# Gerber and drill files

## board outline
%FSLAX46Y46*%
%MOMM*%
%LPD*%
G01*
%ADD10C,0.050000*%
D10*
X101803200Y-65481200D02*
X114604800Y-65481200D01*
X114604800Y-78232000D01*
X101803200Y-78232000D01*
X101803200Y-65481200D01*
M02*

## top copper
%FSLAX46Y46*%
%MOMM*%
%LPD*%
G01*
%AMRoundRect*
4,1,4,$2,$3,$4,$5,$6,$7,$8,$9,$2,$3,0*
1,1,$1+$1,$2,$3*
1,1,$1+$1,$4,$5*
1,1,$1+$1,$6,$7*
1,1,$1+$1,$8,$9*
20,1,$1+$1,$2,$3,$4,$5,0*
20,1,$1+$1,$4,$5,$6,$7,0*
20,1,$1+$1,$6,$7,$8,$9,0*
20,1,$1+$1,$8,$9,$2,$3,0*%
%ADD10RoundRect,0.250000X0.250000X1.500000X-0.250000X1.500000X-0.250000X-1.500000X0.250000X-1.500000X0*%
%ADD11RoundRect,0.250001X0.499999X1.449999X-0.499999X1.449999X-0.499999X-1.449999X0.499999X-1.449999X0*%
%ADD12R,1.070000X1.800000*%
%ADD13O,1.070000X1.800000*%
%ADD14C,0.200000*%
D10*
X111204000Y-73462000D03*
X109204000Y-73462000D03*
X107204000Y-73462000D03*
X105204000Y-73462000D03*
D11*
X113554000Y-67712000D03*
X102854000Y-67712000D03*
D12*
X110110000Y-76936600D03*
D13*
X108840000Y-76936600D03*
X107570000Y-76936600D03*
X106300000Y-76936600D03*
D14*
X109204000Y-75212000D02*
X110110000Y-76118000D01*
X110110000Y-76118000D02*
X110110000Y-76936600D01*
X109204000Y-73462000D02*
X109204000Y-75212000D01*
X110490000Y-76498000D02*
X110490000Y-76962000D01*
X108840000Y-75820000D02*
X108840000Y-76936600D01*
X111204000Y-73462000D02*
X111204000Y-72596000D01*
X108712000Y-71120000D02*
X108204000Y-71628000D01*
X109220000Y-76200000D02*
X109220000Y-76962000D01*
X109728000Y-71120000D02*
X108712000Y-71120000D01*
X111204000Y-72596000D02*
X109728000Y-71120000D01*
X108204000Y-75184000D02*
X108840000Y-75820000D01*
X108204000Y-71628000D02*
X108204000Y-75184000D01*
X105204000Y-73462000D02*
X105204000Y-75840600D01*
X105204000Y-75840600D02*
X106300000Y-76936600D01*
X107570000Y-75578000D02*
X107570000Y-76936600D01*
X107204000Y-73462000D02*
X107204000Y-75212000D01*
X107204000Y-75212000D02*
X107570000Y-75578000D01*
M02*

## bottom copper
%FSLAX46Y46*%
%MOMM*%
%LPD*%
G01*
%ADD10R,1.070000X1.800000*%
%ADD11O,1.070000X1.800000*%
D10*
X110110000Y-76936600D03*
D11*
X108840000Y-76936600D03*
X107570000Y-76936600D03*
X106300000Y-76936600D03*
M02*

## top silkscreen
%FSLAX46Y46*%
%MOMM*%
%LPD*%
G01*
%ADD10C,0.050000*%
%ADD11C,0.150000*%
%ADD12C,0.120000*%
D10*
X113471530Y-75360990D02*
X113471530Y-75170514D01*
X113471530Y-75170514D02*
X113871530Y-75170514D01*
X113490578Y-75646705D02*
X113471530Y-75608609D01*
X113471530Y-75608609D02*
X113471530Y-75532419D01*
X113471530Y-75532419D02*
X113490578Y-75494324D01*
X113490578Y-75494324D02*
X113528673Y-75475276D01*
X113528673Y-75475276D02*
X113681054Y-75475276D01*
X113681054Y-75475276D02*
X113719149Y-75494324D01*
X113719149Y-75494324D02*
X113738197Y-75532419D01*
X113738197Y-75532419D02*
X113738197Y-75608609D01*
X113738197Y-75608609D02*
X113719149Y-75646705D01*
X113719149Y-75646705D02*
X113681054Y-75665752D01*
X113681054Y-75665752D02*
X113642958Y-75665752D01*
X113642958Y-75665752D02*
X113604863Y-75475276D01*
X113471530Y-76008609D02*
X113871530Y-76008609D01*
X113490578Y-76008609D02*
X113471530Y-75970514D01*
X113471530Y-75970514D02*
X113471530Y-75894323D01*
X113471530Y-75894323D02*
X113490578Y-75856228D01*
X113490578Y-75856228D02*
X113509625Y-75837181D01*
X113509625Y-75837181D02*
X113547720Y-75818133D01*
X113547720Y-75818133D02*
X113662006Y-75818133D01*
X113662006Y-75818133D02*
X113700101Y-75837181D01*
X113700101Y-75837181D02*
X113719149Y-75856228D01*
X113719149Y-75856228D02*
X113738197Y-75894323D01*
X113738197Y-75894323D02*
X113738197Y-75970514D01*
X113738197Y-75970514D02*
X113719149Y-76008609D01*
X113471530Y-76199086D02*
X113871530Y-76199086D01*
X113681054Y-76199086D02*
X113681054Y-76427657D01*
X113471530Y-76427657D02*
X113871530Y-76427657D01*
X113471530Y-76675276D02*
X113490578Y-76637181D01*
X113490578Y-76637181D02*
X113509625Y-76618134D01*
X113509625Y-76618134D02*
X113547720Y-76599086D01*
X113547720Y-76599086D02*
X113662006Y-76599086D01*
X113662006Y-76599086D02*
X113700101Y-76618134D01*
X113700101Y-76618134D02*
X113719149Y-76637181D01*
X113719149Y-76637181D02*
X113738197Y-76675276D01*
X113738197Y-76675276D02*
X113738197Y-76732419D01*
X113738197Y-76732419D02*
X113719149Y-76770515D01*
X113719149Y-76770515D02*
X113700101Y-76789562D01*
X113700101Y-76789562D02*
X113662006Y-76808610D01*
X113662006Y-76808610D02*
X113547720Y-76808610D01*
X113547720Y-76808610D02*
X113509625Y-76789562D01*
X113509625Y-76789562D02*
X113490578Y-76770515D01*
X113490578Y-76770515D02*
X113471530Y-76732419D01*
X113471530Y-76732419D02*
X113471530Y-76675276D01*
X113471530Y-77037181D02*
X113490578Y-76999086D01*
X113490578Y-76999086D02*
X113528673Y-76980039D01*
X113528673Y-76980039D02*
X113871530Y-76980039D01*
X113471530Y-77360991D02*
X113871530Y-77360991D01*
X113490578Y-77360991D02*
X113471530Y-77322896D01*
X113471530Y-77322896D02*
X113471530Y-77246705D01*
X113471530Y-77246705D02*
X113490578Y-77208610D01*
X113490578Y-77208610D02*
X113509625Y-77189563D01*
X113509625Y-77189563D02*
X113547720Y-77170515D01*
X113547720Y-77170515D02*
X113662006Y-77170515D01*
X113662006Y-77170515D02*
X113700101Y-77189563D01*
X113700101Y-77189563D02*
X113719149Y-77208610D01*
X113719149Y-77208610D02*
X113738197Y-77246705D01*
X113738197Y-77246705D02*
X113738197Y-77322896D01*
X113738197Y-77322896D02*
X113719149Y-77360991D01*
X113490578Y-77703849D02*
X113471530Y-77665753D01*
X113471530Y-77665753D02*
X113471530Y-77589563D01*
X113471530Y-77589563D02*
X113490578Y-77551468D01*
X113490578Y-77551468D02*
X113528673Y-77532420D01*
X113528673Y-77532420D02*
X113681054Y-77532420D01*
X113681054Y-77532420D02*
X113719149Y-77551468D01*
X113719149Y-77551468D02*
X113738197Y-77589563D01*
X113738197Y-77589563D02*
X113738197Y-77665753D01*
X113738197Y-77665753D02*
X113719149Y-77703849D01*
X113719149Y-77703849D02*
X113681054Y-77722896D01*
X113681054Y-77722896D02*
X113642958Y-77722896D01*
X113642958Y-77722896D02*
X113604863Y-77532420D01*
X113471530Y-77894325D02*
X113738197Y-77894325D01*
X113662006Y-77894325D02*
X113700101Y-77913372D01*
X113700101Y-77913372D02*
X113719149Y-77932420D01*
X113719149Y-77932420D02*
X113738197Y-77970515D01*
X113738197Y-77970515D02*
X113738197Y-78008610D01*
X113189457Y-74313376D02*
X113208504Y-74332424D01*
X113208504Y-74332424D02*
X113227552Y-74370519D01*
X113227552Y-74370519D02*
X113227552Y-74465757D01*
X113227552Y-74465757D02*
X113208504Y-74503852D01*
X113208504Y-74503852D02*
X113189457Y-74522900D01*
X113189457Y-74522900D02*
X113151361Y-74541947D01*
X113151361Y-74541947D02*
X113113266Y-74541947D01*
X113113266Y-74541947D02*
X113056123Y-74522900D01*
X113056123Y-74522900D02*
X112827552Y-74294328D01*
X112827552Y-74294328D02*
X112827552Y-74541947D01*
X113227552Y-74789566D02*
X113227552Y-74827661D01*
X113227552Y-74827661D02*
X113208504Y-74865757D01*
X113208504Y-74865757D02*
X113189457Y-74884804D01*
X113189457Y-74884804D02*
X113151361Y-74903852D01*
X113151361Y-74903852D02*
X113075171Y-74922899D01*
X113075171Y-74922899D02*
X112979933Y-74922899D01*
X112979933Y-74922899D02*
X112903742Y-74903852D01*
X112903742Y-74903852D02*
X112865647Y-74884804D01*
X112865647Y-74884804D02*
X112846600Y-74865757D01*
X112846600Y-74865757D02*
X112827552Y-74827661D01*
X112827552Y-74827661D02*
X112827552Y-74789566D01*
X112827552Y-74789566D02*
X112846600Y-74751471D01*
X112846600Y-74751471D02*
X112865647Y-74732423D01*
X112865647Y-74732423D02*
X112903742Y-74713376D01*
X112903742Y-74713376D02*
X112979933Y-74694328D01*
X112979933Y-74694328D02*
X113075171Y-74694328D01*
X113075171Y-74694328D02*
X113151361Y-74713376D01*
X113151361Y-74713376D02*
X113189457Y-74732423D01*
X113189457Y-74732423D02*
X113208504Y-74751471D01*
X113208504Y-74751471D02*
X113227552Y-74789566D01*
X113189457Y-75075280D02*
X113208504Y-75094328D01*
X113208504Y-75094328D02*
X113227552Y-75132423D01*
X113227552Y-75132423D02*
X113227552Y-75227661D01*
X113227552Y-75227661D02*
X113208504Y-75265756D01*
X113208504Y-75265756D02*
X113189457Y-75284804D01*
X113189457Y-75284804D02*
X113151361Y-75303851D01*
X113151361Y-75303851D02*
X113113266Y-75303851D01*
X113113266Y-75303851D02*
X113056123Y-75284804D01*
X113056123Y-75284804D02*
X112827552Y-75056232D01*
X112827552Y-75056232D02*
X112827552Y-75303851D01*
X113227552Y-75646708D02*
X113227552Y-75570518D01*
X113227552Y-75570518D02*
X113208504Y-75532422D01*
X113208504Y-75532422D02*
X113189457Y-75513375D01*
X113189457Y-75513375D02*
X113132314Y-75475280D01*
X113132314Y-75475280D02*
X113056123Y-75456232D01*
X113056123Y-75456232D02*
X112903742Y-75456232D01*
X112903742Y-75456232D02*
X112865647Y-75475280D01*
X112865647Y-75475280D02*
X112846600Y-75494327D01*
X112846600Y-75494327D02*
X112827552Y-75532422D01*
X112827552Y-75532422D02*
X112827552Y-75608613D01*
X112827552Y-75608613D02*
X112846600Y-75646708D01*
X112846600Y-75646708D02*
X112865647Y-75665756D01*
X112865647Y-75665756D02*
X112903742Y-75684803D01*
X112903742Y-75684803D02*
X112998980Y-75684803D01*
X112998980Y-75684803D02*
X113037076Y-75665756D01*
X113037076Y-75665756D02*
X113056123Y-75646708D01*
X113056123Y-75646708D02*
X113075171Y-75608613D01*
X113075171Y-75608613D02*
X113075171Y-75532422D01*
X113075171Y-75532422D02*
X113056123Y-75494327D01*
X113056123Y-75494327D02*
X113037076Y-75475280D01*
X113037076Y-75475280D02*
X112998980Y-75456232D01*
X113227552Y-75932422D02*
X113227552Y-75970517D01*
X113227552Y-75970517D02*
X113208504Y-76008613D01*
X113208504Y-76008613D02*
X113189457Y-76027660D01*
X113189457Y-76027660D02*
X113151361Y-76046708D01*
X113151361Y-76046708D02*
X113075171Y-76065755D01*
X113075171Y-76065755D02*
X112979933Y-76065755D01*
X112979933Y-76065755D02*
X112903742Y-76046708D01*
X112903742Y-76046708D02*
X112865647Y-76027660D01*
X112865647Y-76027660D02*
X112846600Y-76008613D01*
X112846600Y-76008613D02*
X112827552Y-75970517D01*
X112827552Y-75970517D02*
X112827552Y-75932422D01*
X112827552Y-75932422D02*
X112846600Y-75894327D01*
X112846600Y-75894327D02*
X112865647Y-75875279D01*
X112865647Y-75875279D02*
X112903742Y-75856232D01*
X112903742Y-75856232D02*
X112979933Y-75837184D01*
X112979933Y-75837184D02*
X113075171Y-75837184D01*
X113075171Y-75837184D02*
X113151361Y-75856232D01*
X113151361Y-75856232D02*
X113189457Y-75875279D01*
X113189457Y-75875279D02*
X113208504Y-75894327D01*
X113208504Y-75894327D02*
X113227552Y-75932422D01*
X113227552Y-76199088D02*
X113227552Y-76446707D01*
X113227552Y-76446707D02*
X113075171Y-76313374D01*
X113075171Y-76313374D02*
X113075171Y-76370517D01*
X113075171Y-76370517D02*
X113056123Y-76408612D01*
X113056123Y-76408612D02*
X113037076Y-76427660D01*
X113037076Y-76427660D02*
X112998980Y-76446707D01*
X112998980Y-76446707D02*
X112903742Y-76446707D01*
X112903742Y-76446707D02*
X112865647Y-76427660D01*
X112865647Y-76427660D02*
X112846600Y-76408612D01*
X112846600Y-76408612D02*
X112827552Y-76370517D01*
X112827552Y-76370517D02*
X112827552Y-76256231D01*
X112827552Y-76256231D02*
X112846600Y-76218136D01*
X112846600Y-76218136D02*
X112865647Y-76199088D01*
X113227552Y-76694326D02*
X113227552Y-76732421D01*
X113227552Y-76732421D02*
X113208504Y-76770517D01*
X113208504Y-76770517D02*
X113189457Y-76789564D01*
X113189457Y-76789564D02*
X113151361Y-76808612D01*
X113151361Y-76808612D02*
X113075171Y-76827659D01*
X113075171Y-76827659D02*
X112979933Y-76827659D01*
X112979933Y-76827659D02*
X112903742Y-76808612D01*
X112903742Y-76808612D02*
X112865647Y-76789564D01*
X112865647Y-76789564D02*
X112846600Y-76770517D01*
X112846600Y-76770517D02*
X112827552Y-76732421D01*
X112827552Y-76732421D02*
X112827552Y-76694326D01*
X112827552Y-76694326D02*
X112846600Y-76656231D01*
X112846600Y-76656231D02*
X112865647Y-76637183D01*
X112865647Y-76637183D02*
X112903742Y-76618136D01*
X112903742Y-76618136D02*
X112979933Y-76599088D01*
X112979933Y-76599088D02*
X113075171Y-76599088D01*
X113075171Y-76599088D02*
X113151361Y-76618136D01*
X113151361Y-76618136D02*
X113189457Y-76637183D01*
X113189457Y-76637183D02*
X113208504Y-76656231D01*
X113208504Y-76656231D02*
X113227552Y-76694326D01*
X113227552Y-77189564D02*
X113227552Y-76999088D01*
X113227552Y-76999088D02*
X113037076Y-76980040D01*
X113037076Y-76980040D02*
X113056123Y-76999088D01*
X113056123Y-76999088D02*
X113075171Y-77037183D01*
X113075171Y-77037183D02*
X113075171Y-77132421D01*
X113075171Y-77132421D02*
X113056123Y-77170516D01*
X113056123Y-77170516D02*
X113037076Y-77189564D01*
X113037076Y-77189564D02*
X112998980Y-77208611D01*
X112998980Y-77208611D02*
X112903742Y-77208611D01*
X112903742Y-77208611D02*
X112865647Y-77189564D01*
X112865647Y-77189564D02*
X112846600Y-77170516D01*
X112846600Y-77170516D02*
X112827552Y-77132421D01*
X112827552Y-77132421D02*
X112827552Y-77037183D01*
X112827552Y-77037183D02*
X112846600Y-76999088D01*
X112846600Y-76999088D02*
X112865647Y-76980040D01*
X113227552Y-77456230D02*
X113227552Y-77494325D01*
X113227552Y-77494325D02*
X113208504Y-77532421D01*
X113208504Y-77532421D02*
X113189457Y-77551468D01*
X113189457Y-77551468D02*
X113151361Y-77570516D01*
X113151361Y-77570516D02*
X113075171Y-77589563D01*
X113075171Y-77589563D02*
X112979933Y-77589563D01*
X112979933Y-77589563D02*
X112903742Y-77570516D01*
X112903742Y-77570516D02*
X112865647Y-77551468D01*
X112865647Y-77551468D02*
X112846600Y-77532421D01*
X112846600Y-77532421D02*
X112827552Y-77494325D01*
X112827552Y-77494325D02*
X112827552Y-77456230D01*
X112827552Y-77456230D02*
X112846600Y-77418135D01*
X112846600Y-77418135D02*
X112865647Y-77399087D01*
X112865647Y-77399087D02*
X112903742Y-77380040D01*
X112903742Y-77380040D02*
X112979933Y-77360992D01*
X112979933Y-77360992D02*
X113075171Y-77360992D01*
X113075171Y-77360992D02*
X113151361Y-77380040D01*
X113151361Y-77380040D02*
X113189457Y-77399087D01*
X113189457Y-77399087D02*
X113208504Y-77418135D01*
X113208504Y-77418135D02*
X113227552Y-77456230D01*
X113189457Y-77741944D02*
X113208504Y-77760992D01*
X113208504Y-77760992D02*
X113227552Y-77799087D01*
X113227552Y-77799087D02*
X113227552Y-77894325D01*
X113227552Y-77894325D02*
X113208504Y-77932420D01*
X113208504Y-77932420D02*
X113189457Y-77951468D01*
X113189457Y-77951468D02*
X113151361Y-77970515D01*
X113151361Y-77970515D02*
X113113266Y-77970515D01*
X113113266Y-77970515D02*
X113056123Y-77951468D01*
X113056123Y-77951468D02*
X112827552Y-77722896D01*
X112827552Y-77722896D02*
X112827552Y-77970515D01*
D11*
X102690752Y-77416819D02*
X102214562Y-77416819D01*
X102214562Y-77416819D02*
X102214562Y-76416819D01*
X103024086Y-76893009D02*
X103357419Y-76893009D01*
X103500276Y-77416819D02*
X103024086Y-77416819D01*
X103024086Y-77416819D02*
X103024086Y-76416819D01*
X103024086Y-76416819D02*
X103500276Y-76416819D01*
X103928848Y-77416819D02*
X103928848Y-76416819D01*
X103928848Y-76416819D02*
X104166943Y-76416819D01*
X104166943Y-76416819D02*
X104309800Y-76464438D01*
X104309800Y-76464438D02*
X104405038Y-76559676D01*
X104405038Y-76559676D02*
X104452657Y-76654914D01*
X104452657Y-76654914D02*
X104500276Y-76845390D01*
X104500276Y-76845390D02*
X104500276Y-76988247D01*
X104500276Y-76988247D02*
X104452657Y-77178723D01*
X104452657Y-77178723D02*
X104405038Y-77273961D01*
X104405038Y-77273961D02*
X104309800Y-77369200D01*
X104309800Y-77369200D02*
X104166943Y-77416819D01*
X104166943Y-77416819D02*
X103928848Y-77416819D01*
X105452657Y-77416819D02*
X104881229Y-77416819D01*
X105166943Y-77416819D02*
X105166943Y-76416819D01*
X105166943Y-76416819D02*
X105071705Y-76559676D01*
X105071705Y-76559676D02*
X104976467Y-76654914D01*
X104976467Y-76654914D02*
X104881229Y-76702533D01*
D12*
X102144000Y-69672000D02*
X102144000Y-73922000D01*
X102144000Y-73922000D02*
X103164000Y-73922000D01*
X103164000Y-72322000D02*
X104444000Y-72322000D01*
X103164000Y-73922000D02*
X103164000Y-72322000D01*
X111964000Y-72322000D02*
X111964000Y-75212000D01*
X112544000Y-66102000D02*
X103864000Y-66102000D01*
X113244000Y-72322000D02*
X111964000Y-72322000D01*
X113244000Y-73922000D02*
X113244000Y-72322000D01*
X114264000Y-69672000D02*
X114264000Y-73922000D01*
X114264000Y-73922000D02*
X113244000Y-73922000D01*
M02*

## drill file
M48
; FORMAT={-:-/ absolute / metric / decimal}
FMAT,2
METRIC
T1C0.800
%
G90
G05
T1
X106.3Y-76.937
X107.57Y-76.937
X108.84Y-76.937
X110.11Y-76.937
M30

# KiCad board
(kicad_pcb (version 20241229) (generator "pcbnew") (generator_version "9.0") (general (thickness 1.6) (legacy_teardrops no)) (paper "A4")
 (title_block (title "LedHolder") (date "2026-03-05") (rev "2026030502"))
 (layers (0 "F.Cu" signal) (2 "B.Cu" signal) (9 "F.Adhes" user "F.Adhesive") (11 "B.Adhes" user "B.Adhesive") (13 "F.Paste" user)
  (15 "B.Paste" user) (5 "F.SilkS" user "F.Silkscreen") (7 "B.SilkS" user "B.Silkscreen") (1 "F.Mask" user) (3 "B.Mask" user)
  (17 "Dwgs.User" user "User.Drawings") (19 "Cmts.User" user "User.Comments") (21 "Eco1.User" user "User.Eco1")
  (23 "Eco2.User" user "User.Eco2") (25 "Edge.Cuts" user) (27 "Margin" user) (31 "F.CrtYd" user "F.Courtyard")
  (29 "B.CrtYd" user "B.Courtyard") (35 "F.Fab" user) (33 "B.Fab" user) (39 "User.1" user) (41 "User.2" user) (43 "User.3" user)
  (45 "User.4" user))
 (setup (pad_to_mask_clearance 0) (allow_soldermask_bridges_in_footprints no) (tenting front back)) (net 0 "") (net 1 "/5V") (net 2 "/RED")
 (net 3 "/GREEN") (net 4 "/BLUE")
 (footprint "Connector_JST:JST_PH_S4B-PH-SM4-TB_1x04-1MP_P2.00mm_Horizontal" (layer "F.Cu") (at 108.204 70.612 180)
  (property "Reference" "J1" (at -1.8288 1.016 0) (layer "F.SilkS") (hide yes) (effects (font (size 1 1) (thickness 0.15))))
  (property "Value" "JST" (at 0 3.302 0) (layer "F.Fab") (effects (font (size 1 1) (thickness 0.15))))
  (fp_line (start 6.06 0.94) (end 6.06 -3.31) (stroke (width 0.12) (type solid)) (layer "F.SilkS"))
  (fp_line (start 6.06 -3.31) (end 5.04 -3.31) (stroke (width 0.12) (type solid)) (layer "F.SilkS"))
  (fp_line (start 5.04 -1.71) (end 3.76 -1.71) (stroke (width 0.12) (type solid)) (layer "F.SilkS"))
  (fp_line (start 5.04 -3.31) (end 5.04 -1.71) (stroke (width 0.12) (type solid)) (layer "F.SilkS"))
  (fp_line (start -3.76 -1.71) (end -3.76 -4.6) (stroke (width 0.12) (type solid)) (layer "F.SilkS"))
  (fp_line (start -4.34 4.51) (end 4.34 4.51) (stroke (width 0.12) (type solid)) (layer "F.SilkS"))
  (fp_line (start -5.04 -1.71) (end -3.76 -1.71) (stroke (width 0.12) (type solid)) (layer "F.SilkS"))
  (fp_line (start -5.04 -3.31) (end -5.04 -1.71) (stroke (width 0.12) (type solid)) (layer "F.SilkS"))
  (fp_line (start -6.06 0.94) (end -6.06 -3.31) (stroke (width 0.12) (type solid)) (layer "F.SilkS"))
  (fp_line (start -6.06 -3.31) (end -5.04 -3.31) (stroke (width 0.12) (type solid)) (layer "F.SilkS"))
  (pad "1" smd roundrect (at -3 -2.85 180) (size 1 3.5) (layers "F.Cu" "F.Mask" "F.Paste") (roundrect_rratio 0.25) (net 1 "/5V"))
  (pad "2" smd roundrect (at -1 -2.85 180) (size 1 3.5) (layers "F.Cu" "F.Mask" "F.Paste") (roundrect_rratio 0.25) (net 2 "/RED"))
  (pad "3" smd roundrect (at 1 -2.85 180) (size 1 3.5) (layers "F.Cu" "F.Mask" "F.Paste") (roundrect_rratio 0.25) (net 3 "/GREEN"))
  (pad "4" smd roundrect (at 3 -2.85 180) (size 1 3.5) (layers "F.Cu" "F.Mask" "F.Paste") (roundrect_rratio 0.25) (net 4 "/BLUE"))
  (pad "MP" smd roundrect (at -5.35 2.9 180) (size 1.5 3.4) (layers "F.Cu" "F.Mask" "F.Paste") (roundrect_rratio 0.166667))
  (pad "MP" smd roundrect (at 5.35 2.9 180) (size 1.5 3.4) (layers "F.Cu" "F.Mask" "F.Paste") (roundrect_rratio 0.166667)))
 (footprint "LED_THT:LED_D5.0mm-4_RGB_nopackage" (layer "F.Cu") (at 110.11 76.9366 180)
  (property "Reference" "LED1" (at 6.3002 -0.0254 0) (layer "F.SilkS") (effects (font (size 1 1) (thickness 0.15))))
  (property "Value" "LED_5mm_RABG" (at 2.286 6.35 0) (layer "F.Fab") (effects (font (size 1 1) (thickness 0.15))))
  (pad "1" thru_hole rect (at 0 0 180) (size 1.07 1.8) (drill 0.8) (layers "*.Cu" "*.Mask") (remove_unused_layers no) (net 2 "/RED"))
  (pad "2" thru_hole oval (at 1.27 0 180) (size 1.07 1.8) (drill 0.8) (layers "*.Cu" "*.Mask") (remove_unused_layers no) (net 1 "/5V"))
  (pad "3" thru_hole oval (at 2.54 0 180) (size 1.07 1.8) (drill 0.8) (layers "*.Cu" "*.Mask") (remove_unused_layers no) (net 3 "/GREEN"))
  (pad "4" thru_hole oval (at 3.81 0 180) (size 1.07 1.8) (drill 0.8) (layers "*.Cu" "*.Mask") (remove_unused_layers no) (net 4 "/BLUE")))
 (gr_rect (start 101.8032 65.4812) (end 114.6048 78.232) (stroke (width 0.05) (type default)) (fill no) (layer "Edge.Cuts"))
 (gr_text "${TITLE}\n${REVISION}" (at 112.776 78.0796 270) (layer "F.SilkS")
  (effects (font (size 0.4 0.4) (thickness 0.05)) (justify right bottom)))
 (segment (start 109.204 75.212) (end 110.11 76.118) (width 0.2) (layer "F.Cu") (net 2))
 (segment (start 110.11 76.118) (end 110.11 76.9366) (width 0.2) (layer "F.Cu") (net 2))
 (segment (start 109.204 73.462) (end 109.204 75.212) (width 0.2) (layer "F.Cu") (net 2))
 (segment (start 110.49 76.498) (end 110.49 76.962) (width 0.2) (layer "F.Cu") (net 2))
 (segment (start 108.84 75.82) (end 108.84 76.9366) (width 0.2) (layer "F.Cu") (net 1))
 (segment (start 111.204 73.462) (end 111.204 72.596) (width 0.2) (layer "F.Cu") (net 1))
 (segment (start 108.712 71.12) (end 108.204 71.628) (width 0.2) (layer "F.Cu") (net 1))
 (segment (start 109.22 76.2) (end 109.22 76.962) (width 0.2) (layer "F.Cu") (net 1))
 (segment (start 109.728 71.12) (end 108.712 71.12) (width 0.2) (layer "F.Cu") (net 1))
 (segment (start 111.204 72.596) (end 109.728 71.12) (width 0.2) (layer "F.Cu") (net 1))
 (segment (start 108.204 75.184) (end 108.84 75.82) (width 0.2) (layer "F.Cu") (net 1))
 (segment (start 108.204 71.628) (end 108.204 75.184) (width 0.2) (layer "F.Cu") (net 1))
 (segment (start 105.204 73.462) (end 105.204 75.8406) (width 0.2) (layer "F.Cu") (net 4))
 (segment (start 105.204 75.8406) (end 106.3 76.9366) (width 0.2) (layer "F.Cu") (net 4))
 (segment (start 107.57 75.578) (end 107.57 76.9366) (width 0.2) (layer "F.Cu") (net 3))
 (segment (start 107.204 73.462) (end 107.204 75.212) (width 0.2) (layer "F.Cu") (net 3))
 (segment (start 107.204 75.212) (end 107.57 75.578) (width 0.2) (layer "F.Cu") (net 3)))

